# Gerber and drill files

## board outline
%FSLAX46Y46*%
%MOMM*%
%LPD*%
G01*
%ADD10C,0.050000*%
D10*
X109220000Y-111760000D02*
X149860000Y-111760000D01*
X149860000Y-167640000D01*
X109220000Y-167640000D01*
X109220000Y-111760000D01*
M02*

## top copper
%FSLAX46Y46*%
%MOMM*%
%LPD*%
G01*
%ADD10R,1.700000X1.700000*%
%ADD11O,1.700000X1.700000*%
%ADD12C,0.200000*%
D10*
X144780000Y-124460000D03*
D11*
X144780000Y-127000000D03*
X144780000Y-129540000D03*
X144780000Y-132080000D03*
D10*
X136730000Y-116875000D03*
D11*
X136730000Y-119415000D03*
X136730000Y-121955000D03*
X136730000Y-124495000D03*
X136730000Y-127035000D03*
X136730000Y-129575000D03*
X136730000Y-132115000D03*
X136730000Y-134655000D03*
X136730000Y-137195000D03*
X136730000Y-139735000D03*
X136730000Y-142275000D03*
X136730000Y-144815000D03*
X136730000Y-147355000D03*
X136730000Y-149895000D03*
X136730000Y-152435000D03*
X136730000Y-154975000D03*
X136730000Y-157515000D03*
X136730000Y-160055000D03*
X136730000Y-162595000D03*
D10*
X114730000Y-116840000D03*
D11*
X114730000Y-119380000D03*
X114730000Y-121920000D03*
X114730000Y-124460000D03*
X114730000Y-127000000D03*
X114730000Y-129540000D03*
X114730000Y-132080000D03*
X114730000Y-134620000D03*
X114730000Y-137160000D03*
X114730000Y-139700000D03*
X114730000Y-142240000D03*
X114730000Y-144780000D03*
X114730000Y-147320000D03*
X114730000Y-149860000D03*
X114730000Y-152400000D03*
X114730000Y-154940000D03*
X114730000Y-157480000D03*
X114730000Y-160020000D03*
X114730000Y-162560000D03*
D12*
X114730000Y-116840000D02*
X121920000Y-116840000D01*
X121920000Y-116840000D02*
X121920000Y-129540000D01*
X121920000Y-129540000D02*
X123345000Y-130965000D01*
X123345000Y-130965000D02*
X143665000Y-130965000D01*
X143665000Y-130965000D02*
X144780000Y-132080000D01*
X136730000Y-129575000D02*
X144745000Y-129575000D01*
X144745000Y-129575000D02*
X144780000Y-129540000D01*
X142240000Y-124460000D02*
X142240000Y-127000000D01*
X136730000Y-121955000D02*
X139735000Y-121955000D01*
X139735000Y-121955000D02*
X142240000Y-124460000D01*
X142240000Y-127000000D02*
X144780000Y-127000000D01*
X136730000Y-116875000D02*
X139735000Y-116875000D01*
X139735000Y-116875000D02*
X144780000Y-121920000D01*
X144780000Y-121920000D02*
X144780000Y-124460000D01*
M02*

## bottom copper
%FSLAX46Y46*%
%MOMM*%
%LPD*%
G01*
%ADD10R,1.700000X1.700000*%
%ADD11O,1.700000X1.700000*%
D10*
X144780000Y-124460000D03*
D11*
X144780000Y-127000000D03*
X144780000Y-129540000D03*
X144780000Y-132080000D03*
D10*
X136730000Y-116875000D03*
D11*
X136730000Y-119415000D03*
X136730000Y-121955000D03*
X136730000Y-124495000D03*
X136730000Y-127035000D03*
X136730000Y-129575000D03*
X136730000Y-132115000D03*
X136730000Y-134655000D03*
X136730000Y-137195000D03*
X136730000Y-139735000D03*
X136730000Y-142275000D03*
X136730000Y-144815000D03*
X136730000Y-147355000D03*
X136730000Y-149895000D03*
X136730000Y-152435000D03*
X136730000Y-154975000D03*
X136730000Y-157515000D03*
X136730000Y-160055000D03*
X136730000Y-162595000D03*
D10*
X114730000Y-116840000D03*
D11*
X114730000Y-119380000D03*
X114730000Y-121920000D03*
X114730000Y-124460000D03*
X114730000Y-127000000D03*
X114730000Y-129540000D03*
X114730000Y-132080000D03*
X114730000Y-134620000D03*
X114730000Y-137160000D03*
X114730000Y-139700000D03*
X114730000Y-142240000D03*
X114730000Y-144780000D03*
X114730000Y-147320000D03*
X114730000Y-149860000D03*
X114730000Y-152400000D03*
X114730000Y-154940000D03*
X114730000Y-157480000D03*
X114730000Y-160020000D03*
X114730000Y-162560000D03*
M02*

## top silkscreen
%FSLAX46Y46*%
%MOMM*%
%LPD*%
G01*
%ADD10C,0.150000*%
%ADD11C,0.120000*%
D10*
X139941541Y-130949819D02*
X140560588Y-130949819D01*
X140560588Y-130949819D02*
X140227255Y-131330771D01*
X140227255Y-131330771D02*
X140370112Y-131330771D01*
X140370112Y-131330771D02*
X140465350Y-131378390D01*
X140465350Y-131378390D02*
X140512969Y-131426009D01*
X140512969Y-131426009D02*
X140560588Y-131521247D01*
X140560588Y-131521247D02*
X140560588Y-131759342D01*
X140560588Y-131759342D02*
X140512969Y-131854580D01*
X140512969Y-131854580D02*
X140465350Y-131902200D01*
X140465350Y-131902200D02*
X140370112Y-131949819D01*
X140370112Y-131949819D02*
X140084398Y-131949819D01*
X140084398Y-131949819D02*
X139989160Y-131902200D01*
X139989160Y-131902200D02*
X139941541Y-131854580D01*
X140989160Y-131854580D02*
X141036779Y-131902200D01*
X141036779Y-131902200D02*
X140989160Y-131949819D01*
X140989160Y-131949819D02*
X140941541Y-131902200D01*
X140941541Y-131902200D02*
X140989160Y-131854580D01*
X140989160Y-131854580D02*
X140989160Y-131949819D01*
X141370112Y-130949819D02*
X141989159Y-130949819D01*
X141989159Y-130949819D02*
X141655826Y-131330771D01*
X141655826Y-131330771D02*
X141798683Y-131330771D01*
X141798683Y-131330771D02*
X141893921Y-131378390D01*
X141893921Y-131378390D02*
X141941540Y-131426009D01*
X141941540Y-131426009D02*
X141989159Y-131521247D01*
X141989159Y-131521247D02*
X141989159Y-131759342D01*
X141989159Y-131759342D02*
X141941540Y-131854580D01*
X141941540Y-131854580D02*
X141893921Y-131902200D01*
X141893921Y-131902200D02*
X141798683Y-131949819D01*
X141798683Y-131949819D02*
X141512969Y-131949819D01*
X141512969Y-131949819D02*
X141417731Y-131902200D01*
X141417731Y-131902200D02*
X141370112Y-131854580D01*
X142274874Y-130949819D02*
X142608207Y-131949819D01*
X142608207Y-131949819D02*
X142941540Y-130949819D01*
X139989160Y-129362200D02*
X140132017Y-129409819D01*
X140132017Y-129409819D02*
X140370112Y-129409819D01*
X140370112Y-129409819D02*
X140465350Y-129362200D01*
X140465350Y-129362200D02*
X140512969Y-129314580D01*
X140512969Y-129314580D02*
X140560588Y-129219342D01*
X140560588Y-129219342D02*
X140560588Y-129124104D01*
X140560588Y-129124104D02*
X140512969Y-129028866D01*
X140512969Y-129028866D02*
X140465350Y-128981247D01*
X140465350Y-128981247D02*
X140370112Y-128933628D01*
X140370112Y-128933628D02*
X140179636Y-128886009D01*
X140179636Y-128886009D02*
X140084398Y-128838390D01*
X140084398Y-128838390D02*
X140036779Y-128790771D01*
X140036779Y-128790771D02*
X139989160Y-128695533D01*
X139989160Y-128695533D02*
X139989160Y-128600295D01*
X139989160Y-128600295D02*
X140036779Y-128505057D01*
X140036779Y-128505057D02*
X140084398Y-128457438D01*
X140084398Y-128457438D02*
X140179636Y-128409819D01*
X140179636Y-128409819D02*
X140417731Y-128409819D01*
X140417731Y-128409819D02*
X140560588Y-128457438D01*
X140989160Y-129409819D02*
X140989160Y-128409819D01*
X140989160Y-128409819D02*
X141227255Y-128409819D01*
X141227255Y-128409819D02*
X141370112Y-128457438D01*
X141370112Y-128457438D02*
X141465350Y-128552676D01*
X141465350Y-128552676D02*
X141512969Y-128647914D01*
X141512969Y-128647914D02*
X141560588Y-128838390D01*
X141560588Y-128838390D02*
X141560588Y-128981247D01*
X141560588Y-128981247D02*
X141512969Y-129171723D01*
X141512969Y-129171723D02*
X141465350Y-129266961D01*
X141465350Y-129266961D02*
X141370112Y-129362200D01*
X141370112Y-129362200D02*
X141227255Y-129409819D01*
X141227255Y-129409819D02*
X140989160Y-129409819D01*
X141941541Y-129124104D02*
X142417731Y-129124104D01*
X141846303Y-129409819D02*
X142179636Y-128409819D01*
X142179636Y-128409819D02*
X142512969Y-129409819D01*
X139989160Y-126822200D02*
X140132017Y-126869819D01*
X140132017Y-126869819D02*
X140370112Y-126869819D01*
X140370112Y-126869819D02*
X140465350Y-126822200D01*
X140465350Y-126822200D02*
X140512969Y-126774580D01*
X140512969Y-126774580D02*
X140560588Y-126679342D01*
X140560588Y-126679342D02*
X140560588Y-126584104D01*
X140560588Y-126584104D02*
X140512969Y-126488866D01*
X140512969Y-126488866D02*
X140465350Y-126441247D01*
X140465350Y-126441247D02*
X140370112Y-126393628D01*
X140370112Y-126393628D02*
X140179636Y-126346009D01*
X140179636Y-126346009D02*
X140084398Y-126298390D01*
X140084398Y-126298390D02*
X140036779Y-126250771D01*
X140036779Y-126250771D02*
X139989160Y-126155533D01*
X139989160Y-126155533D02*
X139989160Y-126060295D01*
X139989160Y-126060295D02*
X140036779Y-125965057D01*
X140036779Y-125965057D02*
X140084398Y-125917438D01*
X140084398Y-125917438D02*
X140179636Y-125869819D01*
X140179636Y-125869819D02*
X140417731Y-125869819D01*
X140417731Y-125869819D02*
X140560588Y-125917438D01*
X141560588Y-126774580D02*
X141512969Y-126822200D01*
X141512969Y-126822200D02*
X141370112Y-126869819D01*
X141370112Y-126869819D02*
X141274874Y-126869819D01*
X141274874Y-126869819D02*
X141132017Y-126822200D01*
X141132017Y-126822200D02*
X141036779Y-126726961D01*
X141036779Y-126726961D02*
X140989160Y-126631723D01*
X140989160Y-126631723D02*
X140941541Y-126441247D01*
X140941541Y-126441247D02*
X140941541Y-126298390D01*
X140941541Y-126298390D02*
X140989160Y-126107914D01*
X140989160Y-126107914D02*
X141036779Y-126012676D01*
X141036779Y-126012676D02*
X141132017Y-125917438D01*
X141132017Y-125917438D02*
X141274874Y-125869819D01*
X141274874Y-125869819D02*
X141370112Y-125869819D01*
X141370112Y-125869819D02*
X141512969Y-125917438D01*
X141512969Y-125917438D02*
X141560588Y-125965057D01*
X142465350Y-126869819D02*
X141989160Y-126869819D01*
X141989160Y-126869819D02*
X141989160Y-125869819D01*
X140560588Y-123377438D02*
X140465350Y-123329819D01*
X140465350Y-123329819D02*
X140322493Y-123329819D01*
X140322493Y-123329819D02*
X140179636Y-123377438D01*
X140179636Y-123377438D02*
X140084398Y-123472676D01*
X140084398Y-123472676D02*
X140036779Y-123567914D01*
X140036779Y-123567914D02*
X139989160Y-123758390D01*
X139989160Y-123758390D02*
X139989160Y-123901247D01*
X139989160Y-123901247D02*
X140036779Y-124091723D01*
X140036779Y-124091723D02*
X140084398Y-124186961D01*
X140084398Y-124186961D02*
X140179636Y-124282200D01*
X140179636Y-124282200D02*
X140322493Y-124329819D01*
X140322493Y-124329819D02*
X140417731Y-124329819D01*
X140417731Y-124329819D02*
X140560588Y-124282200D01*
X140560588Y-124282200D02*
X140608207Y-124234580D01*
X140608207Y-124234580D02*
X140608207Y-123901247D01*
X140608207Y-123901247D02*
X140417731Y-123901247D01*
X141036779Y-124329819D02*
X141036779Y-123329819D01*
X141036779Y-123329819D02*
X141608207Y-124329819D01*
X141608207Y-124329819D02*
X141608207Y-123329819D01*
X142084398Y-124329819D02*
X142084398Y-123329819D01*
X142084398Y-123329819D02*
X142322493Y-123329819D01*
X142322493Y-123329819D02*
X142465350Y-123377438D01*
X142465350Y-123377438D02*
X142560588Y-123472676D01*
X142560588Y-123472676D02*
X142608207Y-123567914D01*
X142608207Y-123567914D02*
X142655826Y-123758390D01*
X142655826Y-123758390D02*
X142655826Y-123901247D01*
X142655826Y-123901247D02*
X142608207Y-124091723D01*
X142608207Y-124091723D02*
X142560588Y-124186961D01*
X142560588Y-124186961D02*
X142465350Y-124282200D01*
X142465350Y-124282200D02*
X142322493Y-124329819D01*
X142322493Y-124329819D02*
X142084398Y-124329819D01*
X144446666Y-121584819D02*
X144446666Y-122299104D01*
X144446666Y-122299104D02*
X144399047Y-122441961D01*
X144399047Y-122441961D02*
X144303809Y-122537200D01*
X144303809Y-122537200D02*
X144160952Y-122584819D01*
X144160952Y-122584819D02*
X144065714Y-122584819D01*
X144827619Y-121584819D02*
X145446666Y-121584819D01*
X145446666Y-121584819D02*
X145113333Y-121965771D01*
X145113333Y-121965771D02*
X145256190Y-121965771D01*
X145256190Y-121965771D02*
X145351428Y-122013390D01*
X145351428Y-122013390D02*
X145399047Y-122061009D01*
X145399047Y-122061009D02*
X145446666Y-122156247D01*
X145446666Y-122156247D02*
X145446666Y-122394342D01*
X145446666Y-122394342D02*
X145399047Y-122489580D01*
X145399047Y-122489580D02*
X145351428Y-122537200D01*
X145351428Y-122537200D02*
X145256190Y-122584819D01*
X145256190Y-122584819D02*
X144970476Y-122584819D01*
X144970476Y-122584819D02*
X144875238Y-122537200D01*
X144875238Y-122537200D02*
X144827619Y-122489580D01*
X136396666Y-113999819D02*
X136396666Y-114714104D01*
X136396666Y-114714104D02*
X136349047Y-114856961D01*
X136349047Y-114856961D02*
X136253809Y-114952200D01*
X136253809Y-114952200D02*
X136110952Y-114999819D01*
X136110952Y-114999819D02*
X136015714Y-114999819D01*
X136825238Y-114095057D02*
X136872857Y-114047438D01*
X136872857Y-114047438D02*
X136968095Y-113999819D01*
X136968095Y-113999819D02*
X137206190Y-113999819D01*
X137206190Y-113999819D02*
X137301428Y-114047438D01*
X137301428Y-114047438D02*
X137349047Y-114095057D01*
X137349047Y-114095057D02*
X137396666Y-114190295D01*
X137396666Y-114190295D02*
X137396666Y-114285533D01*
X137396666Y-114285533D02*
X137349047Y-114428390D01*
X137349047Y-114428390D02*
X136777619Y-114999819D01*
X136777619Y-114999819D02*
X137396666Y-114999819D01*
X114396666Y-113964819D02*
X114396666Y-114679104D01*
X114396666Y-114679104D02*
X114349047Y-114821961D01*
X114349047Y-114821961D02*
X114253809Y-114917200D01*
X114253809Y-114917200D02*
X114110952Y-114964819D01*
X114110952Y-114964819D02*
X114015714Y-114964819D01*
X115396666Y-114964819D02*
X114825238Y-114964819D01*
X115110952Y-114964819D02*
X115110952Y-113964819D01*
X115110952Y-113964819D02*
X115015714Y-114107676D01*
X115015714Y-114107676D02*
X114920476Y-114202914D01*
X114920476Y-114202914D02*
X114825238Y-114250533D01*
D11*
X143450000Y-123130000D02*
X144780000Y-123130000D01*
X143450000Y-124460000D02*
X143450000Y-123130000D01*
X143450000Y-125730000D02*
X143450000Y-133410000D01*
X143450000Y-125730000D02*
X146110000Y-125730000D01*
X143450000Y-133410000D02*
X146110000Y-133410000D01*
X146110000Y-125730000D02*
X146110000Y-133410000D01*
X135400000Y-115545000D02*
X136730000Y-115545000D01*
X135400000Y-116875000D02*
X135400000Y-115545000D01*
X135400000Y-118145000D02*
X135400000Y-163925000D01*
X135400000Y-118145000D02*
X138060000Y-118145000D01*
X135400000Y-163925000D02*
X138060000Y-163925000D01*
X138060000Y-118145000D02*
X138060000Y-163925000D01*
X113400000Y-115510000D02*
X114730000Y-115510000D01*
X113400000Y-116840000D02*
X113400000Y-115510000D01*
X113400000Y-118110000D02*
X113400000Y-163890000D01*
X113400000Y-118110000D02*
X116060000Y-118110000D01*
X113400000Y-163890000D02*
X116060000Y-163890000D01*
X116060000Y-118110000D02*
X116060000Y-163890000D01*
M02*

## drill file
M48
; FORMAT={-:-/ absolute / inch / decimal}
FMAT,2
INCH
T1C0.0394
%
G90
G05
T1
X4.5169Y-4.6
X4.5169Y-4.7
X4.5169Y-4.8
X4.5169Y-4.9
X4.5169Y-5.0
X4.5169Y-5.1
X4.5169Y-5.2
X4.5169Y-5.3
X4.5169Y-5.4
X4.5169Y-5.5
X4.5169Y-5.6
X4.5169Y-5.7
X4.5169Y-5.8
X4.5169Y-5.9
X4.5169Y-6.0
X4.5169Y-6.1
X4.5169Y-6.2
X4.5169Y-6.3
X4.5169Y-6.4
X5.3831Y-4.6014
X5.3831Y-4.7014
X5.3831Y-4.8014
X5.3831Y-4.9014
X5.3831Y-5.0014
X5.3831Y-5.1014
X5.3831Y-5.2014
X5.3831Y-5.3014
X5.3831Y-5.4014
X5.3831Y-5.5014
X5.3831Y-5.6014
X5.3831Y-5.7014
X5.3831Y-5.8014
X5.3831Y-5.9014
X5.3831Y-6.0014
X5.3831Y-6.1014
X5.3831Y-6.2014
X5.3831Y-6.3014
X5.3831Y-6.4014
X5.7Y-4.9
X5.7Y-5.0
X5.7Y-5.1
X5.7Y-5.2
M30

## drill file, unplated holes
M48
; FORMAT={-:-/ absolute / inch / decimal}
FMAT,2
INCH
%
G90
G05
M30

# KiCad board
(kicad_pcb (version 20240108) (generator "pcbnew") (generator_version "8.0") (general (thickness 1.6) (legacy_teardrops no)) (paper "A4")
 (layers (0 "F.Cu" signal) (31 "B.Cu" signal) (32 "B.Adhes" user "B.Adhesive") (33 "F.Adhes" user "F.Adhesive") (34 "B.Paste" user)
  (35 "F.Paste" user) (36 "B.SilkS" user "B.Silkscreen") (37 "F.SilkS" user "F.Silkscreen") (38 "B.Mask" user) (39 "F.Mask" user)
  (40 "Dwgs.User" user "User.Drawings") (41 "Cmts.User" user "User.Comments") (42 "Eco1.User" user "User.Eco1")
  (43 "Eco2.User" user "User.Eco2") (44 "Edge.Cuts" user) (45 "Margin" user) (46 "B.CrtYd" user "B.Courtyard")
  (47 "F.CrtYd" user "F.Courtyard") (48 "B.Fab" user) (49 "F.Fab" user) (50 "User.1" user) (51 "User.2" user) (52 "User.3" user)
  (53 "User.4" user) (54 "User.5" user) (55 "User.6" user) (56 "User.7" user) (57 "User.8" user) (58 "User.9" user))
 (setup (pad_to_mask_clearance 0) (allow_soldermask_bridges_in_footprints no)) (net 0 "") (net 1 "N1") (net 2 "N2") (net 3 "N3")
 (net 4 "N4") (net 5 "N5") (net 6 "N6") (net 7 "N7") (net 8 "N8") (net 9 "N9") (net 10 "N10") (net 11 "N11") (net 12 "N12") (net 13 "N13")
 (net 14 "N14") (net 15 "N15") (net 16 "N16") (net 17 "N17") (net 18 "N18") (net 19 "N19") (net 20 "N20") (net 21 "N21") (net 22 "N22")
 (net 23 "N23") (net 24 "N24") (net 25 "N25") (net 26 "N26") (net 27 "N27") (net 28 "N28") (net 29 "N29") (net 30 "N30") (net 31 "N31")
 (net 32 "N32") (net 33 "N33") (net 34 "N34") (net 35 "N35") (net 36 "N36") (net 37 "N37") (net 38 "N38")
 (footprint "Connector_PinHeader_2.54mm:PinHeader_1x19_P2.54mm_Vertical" (layer "F.Cu") (at 114.73 116.84)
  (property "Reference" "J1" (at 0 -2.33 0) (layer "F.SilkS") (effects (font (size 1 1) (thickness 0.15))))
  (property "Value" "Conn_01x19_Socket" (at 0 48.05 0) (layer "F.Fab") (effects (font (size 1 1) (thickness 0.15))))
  (fp_line (start -1.33 -1.33) (end 0 -1.33) (stroke (width 0.12) (type solid)) (layer "F.SilkS"))
  (fp_line (start -1.33 0) (end -1.33 -1.33) (stroke (width 0.12) (type solid)) (layer "F.SilkS"))
  (fp_line (start -1.33 1.27) (end -1.33 47.05) (stroke (width 0.12) (type solid)) (layer "F.SilkS"))
  (fp_line (start -1.33 1.27) (end 1.33 1.27) (stroke (width 0.12) (type solid)) (layer "F.SilkS"))
  (fp_line (start -1.33 47.05) (end 1.33 47.05) (stroke (width 0.12) (type solid)) (layer "F.SilkS"))
  (fp_line (start 1.33 1.27) (end 1.33 47.05) (stroke (width 0.12) (type solid)) (layer "F.SilkS"))
  (pad "1" thru_hole rect (at 0 0) (size 1.7 1.7) (drill 1) (layers "*.Cu" "*.Mask") (remove_unused_layers no) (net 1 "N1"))
  (pad "2" thru_hole oval (at 0 2.54) (size 1.7 1.7) (drill 1) (layers "*.Cu" "*.Mask") (remove_unused_layers no) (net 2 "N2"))
  (pad "3" thru_hole oval (at 0 5.08) (size 1.7 1.7) (drill 1) (layers "*.Cu" "*.Mask") (remove_unused_layers no) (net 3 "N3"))
  (pad "4" thru_hole oval (at 0 7.62) (size 1.7 1.7) (drill 1) (layers "*.Cu" "*.Mask") (remove_unused_layers no) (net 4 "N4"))
  (pad "5" thru_hole oval (at 0 10.16) (size 1.7 1.7) (drill 1) (layers "*.Cu" "*.Mask") (remove_unused_layers no) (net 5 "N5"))
  (pad "6" thru_hole oval (at 0 12.7) (size 1.7 1.7) (drill 1) (layers "*.Cu" "*.Mask") (remove_unused_layers no) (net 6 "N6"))
  (pad "7" thru_hole oval (at 0 15.24) (size 1.7 1.7) (drill 1) (layers "*.Cu" "*.Mask") (remove_unused_layers no) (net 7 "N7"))
  (pad "8" thru_hole oval (at 0 17.78) (size 1.7 1.7) (drill 1) (layers "*.Cu" "*.Mask") (remove_unused_layers no) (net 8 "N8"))
  (pad "9" thru_hole oval (at 0 20.32) (size 1.7 1.7) (drill 1) (layers "*.Cu" "*.Mask") (remove_unused_layers no) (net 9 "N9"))
  (pad "10" thru_hole oval (at 0 22.86) (size 1.7 1.7) (drill 1) (layers "*.Cu" "*.Mask") (remove_unused_layers no) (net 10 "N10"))
  (pad "11" thru_hole oval (at 0 25.4) (size 1.7 1.7) (drill 1) (layers "*.Cu" "*.Mask") (remove_unused_layers no) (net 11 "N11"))
  (pad "12" thru_hole oval (at 0 27.94) (size 1.7 1.7) (drill 1) (layers "*.Cu" "*.Mask") (remove_unused_layers no) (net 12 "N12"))
  (pad "13" thru_hole oval (at 0 30.48) (size 1.7 1.7) (drill 1) (layers "*.Cu" "*.Mask") (remove_unused_layers no) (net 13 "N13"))
  (pad "14" thru_hole oval (at 0 33.02) (size 1.7 1.7) (drill 1) (layers "*.Cu" "*.Mask") (remove_unused_layers no) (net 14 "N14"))
  (pad "15" thru_hole oval (at 0 35.56) (size 1.7 1.7) (drill 1) (layers "*.Cu" "*.Mask") (remove_unused_layers no) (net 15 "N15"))
  (pad "16" thru_hole oval (at 0 38.1) (size 1.7 1.7) (drill 1) (layers "*.Cu" "*.Mask") (remove_unused_layers no) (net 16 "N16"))
  (pad "17" thru_hole oval (at 0 40.64) (size 1.7 1.7) (drill 1) (layers "*.Cu" "*.Mask") (remove_unused_layers no) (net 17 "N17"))
  (pad "18" thru_hole oval (at 0 43.18) (size 1.7 1.7) (drill 1) (layers "*.Cu" "*.Mask") (remove_unused_layers no) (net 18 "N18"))
  (pad "19" thru_hole oval (at 0 45.72) (size 1.7 1.7) (drill 1) (layers "*.Cu" "*.Mask") (remove_unused_layers no) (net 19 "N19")))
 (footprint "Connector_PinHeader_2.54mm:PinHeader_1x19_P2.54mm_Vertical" (layer "F.Cu") (at 136.73 116.875)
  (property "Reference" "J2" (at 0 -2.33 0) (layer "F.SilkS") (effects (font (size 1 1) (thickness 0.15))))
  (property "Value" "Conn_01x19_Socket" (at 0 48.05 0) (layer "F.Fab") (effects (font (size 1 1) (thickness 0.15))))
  (fp_line (start -1.33 -1.33) (end 0 -1.33) (stroke (width 0.12) (type solid)) (layer "F.SilkS"))
  (fp_line (start -1.33 0) (end -1.33 -1.33) (stroke (width 0.12) (type solid)) (layer "F.SilkS"))
  (fp_line (start -1.33 1.27) (end -1.33 47.05) (stroke (width 0.12) (type solid)) (layer "F.SilkS"))
  (fp_line (start -1.33 1.27) (end 1.33 1.27) (stroke (width 0.12) (type solid)) (layer "F.SilkS"))
  (fp_line (start -1.33 47.05) (end 1.33 47.05) (stroke (width 0.12) (type solid)) (layer "F.SilkS"))
  (fp_line (start 1.33 1.27) (end 1.33 47.05) (stroke (width 0.12) (type solid)) (layer "F.SilkS"))
  (pad "1" thru_hole rect (at 0 0) (size 1.7 1.7) (drill 1) (layers "*.Cu" "*.Mask") (remove_unused_layers no) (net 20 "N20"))
  (pad "2" thru_hole oval (at 0 2.54) (size 1.7 1.7) (drill 1) (layers "*.Cu" "*.Mask") (remove_unused_layers no) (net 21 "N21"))
  (pad "3" thru_hole oval (at 0 5.08) (size 1.7 1.7) (drill 1) (layers "*.Cu" "*.Mask") (remove_unused_layers no) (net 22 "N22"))
  (pad "4" thru_hole oval (at 0 7.62) (size 1.7 1.7) (drill 1) (layers "*.Cu" "*.Mask") (remove_unused_layers no) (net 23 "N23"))
  (pad "5" thru_hole oval (at 0 10.16) (size 1.7 1.7) (drill 1) (layers "*.Cu" "*.Mask") (remove_unused_layers no) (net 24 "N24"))
  (pad "6" thru_hole oval (at 0 12.7) (size 1.7 1.7) (drill 1) (layers "*.Cu" "*.Mask") (remove_unused_layers no) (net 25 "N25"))
  (pad "7" thru_hole oval (at 0 15.24) (size 1.7 1.7) (drill 1) (layers "*.Cu" "*.Mask") (remove_unused_layers no) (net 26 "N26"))
  (pad "8" thru_hole oval (at 0 17.78) (size 1.7 1.7) (drill 1) (layers "*.Cu" "*.Mask") (remove_unused_layers no) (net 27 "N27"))
  (pad "9" thru_hole oval (at 0 20.32) (size 1.7 1.7) (drill 1) (layers "*.Cu" "*.Mask") (remove_unused_layers no) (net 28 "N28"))
  (pad "10" thru_hole oval (at 0 22.86) (size 1.7 1.7) (drill 1) (layers "*.Cu" "*.Mask") (remove_unused_layers no) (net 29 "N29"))
  (pad "11" thru_hole oval (at 0 25.4) (size 1.7 1.7) (drill 1) (layers "*.Cu" "*.Mask") (remove_unused_layers no) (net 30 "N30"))
  (pad "12" thru_hole oval (at 0 27.94) (size 1.7 1.7) (drill 1) (layers "*.Cu" "*.Mask") (remove_unused_layers no) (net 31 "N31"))
  (pad "13" thru_hole oval (at 0 30.48) (size 1.7 1.7) (drill 1) (layers "*.Cu" "*.Mask") (remove_unused_layers no) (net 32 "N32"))
  (pad "14" thru_hole oval (at 0 33.02) (size 1.7 1.7) (drill 1) (layers "*.Cu" "*.Mask") (remove_unused_layers no) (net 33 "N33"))
  (pad "15" thru_hole oval (at 0 35.56) (size 1.7 1.7) (drill 1) (layers "*.Cu" "*.Mask") (remove_unused_layers no) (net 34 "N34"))
  (pad "16" thru_hole oval (at 0 38.1) (size 1.7 1.7) (drill 1) (layers "*.Cu" "*.Mask") (remove_unused_layers no) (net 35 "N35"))
  (pad "17" thru_hole oval (at 0 40.64) (size 1.7 1.7) (drill 1) (layers "*.Cu" "*.Mask") (remove_unused_layers no) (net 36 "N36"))
  (pad "18" thru_hole oval (at 0 43.18) (size 1.7 1.7) (drill 1) (layers "*.Cu" "*.Mask") (remove_unused_layers no) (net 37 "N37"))
  (pad "19" thru_hole oval (at 0 45.72) (size 1.7 1.7) (drill 1) (layers "*.Cu" "*.Mask") (remove_unused_layers no) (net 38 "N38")))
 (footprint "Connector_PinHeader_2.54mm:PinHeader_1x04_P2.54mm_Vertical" (layer "F.Cu") (at 144.78 124.46)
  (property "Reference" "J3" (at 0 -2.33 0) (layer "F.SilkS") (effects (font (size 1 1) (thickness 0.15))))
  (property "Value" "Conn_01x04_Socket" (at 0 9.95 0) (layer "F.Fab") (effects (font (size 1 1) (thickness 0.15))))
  (fp_line (start -1.33 -1.33) (end 0 -1.33) (stroke (width 0.12) (type solid)) (layer "F.SilkS"))
  (fp_line (start -1.33 0) (end -1.33 -1.33) (stroke (width 0.12) (type solid)) (layer "F.SilkS"))
  (fp_line (start -1.33 1.27) (end -1.33 8.95) (stroke (width 0.12) (type solid)) (layer "F.SilkS"))
  (fp_line (start -1.33 1.27) (end 1.33 1.27) (stroke (width 0.12) (type solid)) (layer "F.SilkS"))
  (fp_line (start -1.33 8.95) (end 1.33 8.95) (stroke (width 0.12) (type solid)) (layer "F.SilkS"))
  (fp_line (start 1.33 1.27) (end 1.33 8.95) (stroke (width 0.12) (type solid)) (layer "F.SilkS"))
  (pad "1" thru_hole rect (at 0 0) (size 1.7 1.7) (drill 1) (layers "*.Cu" "*.Mask") (remove_unused_layers no) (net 20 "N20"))
  (pad "2" thru_hole oval (at 0 2.54) (size 1.7 1.7) (drill 1) (layers "*.Cu" "*.Mask") (remove_unused_layers no) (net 22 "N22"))
  (pad "3" thru_hole oval (at 0 5.08) (size 1.7 1.7) (drill 1) (layers "*.Cu" "*.Mask") (remove_unused_layers no) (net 25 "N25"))
  (pad "4" thru_hole oval (at 0 7.62) (size 1.7 1.7) (drill 1) (layers "*.Cu" "*.Mask") (remove_unused_layers no) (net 1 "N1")))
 (gr_rect (start 109.22 111.76) (end 149.86 167.64) (stroke (width 0.05) (type default)) (fill none) (layer "Edge.Cuts"))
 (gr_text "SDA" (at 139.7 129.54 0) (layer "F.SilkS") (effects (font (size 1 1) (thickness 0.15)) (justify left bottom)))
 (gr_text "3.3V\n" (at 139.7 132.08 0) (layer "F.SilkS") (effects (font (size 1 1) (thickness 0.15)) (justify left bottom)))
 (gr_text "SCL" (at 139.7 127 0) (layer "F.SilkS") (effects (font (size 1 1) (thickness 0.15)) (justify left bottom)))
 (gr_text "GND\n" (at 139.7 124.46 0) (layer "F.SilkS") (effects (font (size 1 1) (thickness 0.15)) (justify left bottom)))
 (segment (start 121.92 129.54) (end 123.345 130.965) (width 0.2) (layer "F.Cu") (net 1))
 (segment (start 143.665 130.965) (end 144.78 132.08) (width 0.2) (layer "F.Cu") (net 1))
 (segment (start 123.345 130.965) (end 143.665 130.965) (width 0.2) (layer "F.Cu") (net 1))
 (segment (start 114.73 116.84) (end 121.92 116.84) (width 0.2) (layer "F.Cu") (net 1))
 (segment (start 121.92 116.84) (end 121.92 129.54) (width 0.2) (layer "F.Cu") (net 1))
 (segment (start 144.745 129.575) (end 144.78 129.54) (width 0.2) (layer "F.Cu") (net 25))
 (segment (start 136.73 129.575) (end 144.745 129.575) (width 0.2) (layer "F.Cu") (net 25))
 (segment (start 139.735 116.875) (end 144.78 121.92) (width 0.2) (layer "F.Cu") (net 20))
 (segment (start 136.73 116.875) (end 139.735 116.875) (width 0.2) (layer "F.Cu") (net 20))
 (segment (start 144.78 121.92) (end 144.78 124.46) (width 0.2) (layer "F.Cu") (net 20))
 (segment (start 142.24 127) (end 144.78 127) (width 0.2) (layer "F.Cu") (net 22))
 (segment (start 136.73 121.955) (end 139.735 121.955) (width 0.2) (layer "F.Cu") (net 22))
 (segment (start 139.735 121.955) (end 142.24 124.46) (width 0.2) (layer "F.Cu") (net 22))
 (segment (start 142.24 124.46) (end 142.24 127) (width 0.2) (layer "F.Cu") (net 22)))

